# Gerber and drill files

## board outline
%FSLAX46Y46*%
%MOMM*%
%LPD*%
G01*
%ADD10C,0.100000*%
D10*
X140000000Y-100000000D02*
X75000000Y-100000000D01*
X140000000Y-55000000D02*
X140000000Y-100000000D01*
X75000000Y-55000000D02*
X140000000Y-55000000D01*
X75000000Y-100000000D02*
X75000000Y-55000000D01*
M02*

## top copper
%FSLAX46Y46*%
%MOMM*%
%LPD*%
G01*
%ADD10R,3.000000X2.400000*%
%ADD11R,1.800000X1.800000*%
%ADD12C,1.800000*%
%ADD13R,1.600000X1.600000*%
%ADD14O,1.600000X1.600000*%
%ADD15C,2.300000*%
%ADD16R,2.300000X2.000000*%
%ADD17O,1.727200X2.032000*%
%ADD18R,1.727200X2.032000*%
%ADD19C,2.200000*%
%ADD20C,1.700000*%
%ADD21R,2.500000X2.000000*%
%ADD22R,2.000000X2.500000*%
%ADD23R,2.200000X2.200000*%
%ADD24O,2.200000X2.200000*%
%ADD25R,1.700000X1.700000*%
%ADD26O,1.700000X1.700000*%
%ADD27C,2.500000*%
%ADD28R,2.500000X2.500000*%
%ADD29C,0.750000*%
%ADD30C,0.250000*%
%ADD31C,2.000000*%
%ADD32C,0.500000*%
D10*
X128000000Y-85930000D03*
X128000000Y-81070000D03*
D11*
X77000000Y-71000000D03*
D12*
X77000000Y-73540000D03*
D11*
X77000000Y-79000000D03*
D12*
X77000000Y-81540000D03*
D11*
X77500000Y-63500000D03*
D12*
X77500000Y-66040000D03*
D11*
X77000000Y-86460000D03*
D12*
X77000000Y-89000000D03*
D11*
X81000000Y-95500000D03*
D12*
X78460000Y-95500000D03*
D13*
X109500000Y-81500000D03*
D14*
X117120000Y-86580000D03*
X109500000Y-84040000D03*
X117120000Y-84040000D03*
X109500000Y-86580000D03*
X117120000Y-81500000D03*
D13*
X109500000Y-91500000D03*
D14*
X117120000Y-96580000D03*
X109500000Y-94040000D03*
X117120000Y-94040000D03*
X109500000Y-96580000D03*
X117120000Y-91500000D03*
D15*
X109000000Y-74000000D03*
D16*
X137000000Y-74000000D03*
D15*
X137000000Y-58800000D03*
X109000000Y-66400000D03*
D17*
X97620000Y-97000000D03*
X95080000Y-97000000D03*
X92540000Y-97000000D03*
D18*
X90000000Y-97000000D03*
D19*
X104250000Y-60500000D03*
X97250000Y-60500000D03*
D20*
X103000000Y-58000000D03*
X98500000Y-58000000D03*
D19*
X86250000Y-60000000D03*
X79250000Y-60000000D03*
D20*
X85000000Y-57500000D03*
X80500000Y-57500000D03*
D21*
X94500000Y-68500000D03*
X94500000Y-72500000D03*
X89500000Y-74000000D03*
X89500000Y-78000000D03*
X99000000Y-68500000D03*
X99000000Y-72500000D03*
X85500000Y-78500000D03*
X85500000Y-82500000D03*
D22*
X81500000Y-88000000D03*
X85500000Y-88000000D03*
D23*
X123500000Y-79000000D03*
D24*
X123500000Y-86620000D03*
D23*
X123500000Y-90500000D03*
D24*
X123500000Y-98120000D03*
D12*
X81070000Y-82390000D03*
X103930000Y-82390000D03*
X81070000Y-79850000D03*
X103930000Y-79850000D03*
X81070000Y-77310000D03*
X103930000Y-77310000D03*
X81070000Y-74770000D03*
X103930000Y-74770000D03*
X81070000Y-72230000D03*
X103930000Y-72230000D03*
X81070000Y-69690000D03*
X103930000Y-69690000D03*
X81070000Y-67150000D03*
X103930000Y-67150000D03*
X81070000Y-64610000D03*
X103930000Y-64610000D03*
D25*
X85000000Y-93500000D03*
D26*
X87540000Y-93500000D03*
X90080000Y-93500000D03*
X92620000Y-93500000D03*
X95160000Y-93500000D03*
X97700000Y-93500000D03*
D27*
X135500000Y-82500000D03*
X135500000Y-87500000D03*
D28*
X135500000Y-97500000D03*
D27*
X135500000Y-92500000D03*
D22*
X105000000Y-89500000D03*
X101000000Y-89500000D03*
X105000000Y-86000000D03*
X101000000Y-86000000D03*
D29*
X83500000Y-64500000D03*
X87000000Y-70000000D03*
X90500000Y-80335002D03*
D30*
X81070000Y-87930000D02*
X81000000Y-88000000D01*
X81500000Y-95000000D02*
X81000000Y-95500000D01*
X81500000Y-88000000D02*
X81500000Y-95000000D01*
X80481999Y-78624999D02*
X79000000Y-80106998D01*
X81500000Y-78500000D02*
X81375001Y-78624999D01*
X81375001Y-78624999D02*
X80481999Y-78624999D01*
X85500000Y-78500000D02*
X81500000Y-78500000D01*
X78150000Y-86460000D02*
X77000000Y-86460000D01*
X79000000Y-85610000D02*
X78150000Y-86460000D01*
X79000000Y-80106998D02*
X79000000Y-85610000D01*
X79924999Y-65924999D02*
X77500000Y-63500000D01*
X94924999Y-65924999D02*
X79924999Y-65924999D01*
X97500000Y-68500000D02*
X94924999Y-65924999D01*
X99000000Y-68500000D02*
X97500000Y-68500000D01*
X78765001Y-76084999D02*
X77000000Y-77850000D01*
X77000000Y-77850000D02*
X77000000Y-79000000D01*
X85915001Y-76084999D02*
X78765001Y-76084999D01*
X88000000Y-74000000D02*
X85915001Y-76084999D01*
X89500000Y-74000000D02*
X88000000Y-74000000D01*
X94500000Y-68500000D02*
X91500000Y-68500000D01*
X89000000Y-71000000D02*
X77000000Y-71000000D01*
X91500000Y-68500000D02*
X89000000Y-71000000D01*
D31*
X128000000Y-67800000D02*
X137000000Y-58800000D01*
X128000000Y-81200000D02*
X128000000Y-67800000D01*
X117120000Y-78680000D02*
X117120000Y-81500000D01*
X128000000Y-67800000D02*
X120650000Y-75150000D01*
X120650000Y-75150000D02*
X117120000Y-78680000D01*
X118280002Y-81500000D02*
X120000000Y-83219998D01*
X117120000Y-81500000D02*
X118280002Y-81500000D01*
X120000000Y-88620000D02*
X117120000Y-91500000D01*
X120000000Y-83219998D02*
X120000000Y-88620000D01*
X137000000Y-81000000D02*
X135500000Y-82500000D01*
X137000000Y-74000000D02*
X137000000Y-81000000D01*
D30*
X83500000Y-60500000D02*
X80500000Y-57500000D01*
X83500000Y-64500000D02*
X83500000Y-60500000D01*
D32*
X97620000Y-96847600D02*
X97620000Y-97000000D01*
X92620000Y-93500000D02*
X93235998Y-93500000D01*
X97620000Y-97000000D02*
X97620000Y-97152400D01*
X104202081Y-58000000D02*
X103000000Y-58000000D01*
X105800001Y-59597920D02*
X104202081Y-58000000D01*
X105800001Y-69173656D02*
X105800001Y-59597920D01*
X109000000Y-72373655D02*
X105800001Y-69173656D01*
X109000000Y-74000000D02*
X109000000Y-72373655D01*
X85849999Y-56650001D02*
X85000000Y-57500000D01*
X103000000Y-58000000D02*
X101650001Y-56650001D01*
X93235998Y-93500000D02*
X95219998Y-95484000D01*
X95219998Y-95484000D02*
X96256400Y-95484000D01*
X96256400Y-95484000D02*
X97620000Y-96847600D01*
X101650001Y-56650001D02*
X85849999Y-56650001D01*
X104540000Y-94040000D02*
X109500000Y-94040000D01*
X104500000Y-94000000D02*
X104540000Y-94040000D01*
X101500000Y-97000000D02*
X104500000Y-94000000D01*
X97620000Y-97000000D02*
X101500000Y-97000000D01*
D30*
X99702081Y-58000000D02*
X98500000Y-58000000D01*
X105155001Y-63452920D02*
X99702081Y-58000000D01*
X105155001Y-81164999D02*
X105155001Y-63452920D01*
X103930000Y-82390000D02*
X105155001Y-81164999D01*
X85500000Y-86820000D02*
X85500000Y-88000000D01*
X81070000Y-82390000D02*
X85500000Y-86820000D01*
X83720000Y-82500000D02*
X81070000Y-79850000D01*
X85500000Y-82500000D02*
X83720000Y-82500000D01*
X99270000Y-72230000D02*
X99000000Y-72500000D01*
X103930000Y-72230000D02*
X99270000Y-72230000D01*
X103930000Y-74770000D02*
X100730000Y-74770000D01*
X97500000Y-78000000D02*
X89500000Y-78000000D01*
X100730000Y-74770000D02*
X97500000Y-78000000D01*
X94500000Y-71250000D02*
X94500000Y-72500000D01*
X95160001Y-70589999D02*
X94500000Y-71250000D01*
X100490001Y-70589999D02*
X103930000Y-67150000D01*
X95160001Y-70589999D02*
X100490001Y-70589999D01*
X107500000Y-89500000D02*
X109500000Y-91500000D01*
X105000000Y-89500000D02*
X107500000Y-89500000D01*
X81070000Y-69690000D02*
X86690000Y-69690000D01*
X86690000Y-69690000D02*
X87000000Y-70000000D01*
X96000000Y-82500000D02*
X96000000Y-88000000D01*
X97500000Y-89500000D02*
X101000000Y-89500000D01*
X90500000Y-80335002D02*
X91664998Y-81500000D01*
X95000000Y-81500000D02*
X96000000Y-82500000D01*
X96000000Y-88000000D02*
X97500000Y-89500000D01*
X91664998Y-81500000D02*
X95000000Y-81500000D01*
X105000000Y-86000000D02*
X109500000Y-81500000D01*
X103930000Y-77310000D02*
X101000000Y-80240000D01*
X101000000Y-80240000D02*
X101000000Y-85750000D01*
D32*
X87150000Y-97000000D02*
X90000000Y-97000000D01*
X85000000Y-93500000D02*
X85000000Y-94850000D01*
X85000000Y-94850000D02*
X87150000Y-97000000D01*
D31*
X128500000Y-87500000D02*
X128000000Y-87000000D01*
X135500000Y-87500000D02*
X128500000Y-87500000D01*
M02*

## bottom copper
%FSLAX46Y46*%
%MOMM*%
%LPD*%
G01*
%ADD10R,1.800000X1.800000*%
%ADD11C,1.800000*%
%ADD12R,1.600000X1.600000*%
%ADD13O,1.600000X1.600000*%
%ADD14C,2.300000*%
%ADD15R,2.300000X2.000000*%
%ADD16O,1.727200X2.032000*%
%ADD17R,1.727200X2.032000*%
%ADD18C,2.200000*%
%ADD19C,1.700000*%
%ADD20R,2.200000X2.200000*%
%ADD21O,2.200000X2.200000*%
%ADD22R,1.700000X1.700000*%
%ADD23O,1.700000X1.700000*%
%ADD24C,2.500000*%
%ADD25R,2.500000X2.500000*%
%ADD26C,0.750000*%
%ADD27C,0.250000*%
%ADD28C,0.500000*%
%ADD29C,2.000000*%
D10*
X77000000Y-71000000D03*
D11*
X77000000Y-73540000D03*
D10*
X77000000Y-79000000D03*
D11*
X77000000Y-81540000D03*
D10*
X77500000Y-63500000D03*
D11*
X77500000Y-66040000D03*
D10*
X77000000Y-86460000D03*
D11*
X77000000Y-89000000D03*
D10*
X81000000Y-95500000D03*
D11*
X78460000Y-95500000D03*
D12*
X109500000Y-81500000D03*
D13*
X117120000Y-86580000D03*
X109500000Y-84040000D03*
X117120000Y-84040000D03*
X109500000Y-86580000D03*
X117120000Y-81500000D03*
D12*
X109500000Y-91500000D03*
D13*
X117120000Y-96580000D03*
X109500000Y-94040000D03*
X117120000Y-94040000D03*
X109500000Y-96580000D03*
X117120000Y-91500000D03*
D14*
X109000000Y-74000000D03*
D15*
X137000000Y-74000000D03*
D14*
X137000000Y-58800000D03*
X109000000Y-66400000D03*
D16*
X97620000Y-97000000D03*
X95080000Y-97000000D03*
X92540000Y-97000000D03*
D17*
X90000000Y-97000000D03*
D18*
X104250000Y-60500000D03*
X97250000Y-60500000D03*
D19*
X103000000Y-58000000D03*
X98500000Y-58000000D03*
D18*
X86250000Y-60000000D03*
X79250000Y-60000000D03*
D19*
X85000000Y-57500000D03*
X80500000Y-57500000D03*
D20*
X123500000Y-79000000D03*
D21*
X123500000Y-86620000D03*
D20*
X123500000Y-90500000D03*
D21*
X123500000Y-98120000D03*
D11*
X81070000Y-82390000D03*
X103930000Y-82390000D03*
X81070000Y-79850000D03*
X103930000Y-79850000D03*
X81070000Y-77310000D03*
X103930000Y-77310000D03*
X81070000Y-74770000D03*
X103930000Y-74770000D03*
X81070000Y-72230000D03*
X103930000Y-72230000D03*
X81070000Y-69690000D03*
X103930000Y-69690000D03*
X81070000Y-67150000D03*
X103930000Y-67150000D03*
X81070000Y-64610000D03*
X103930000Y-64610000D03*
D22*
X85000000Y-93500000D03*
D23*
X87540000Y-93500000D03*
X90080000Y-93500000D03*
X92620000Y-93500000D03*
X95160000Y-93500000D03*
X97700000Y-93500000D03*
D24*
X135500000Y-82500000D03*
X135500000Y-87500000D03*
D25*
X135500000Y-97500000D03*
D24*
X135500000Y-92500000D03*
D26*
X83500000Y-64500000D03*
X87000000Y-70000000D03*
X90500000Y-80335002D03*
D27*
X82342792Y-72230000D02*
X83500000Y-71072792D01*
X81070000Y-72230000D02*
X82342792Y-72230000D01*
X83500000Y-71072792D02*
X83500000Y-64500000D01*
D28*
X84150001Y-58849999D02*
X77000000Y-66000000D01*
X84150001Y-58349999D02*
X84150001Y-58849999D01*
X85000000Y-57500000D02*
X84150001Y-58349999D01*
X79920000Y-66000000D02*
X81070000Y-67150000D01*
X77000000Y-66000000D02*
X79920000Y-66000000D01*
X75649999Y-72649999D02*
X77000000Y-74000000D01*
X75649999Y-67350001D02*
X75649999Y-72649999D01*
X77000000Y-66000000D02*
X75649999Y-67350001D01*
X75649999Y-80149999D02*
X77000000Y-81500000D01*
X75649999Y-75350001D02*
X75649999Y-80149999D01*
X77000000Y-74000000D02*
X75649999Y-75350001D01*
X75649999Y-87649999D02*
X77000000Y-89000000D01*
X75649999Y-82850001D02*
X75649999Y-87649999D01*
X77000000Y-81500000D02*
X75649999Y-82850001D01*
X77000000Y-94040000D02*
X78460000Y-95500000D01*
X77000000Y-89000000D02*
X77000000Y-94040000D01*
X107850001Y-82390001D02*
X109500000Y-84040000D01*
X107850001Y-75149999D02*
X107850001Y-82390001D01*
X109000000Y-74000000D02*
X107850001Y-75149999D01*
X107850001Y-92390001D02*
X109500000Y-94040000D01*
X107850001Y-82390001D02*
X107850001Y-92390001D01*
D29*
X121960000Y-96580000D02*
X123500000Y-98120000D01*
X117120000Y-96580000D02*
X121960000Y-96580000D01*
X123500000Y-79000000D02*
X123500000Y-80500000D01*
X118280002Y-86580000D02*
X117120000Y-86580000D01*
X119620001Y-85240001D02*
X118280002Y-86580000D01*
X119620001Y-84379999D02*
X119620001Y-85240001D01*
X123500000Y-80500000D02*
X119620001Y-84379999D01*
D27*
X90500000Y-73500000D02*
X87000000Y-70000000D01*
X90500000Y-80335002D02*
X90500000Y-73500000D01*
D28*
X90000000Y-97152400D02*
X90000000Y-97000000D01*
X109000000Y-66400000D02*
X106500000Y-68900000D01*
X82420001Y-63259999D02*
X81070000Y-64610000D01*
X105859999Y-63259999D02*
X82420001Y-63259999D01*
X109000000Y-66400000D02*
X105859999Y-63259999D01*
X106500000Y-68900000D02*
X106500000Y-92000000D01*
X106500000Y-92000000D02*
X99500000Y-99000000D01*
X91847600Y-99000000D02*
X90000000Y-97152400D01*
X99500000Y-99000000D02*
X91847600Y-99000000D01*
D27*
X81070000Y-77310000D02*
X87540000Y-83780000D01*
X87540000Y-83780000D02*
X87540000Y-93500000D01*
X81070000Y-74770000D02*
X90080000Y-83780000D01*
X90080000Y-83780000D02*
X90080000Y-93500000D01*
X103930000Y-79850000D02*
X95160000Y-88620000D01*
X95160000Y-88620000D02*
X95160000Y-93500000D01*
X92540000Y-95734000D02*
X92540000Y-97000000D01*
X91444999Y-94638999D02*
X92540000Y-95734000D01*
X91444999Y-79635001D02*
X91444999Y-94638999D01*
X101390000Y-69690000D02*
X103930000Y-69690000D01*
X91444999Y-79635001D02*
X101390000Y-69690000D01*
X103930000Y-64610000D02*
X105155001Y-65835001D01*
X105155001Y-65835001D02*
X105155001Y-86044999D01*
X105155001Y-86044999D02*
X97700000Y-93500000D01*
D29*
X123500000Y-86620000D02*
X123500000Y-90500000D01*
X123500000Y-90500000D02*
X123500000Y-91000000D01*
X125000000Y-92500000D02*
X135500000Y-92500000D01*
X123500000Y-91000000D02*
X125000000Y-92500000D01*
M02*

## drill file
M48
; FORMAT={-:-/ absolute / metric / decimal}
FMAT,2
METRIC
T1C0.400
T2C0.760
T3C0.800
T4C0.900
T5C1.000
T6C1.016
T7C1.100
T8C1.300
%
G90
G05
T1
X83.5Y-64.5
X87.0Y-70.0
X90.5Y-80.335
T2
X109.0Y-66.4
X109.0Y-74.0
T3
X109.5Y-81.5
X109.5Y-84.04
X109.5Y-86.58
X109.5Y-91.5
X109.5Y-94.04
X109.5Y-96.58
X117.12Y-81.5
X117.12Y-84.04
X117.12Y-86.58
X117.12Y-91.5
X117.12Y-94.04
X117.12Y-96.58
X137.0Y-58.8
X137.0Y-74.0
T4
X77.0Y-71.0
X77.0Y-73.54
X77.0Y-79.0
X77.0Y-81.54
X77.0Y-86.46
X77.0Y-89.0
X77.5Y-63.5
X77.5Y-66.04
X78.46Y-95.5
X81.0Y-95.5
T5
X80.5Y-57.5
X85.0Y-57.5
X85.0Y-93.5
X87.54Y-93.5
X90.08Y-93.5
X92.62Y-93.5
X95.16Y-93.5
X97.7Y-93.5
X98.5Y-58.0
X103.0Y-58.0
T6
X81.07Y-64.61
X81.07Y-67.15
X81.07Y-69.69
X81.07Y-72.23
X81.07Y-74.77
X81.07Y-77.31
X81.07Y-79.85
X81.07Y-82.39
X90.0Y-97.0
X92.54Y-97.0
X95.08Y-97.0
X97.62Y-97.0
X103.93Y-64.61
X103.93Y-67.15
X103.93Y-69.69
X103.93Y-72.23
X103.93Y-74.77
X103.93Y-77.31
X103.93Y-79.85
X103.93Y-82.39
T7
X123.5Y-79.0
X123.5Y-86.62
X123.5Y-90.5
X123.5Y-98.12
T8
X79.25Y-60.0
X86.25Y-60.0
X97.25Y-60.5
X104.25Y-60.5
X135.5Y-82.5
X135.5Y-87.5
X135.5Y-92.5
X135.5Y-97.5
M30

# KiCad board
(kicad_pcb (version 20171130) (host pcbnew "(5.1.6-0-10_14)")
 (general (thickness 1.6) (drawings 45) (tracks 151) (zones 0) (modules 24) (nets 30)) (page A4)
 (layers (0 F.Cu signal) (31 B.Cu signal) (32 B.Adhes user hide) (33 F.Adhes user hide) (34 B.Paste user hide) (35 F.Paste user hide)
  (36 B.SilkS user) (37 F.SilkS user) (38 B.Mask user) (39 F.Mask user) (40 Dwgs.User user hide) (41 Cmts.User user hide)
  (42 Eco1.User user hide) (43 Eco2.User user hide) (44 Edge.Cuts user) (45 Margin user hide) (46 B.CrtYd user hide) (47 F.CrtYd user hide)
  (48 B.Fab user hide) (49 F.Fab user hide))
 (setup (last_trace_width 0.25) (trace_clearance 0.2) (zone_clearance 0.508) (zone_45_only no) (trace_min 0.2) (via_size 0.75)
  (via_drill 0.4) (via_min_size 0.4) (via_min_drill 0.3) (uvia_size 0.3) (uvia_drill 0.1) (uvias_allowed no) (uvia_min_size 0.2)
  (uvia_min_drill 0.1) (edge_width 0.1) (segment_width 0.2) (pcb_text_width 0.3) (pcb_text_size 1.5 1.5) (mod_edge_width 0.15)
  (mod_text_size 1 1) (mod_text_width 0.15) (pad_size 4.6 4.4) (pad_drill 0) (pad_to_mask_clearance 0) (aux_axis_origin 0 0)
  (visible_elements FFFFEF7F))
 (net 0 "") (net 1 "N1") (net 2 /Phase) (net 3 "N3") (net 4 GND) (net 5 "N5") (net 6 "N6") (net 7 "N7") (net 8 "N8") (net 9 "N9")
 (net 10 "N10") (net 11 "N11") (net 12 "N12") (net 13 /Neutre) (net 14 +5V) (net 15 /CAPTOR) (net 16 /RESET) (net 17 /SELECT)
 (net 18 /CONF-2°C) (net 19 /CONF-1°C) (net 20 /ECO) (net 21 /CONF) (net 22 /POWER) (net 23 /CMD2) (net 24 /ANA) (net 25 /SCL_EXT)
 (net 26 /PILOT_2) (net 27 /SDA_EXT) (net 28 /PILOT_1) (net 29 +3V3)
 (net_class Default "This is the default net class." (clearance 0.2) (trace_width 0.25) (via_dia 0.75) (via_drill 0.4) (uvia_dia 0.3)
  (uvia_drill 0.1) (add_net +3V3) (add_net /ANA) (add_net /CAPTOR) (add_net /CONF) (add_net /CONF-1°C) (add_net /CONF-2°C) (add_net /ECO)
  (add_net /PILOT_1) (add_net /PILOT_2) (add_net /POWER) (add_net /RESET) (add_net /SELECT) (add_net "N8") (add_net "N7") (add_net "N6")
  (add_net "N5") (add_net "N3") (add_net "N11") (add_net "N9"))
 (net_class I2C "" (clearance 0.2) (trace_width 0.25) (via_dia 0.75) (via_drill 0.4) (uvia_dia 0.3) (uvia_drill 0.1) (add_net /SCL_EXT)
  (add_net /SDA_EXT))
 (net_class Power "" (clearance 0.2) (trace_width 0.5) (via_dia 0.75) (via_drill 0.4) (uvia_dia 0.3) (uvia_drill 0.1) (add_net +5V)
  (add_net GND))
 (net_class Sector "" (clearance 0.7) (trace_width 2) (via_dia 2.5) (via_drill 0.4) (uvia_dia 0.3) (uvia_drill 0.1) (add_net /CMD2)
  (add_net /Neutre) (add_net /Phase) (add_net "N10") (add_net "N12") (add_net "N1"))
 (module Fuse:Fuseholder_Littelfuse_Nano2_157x (layer F.Cu) (at 128 83.5 270)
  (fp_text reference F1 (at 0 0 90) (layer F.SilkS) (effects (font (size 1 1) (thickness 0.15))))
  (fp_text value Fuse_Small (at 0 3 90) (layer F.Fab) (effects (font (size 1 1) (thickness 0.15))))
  (pad 2 smd rect (at 2.43 0 270) (size 2.4 3) (layers F.Cu F.Paste F.Mask) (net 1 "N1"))
  (pad 1 smd rect (at -2.43 0 270) (size 2.4 3) (layers F.Cu F.Paste F.Mask) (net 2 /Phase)))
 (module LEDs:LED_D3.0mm (layer F.Cu) (at 77 71 270)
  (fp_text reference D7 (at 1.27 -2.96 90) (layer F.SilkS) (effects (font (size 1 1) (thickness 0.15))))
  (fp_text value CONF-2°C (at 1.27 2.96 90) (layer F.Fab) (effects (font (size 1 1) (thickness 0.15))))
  (pad 1 thru_hole rect (at 0 0 270) (size 1.8 1.8) (drill 0.9) (layers *.Cu *.Mask) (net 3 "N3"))
  (pad 2 thru_hole circle (at 2.54 0 270) (size 1.8 1.8) (drill 0.9) (layers *.Cu *.Mask) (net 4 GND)))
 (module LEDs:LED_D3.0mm (layer F.Cu) (at 77 79 270)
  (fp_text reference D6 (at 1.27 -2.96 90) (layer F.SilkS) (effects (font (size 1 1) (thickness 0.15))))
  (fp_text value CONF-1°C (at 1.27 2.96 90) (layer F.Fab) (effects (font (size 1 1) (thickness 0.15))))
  (pad 1 thru_hole rect (at 0 0 270) (size 1.8 1.8) (drill 0.9) (layers *.Cu *.Mask) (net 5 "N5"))
  (pad 2 thru_hole circle (at 2.54 0 270) (size 1.8 1.8) (drill 0.9) (layers *.Cu *.Mask) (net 4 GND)))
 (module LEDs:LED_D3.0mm (layer F.Cu) (at 77.5 63.5 270)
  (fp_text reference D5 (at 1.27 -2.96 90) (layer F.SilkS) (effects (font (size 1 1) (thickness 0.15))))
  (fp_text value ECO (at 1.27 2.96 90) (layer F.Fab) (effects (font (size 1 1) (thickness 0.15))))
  (pad 1 thru_hole rect (at 0 0 270) (size 1.8 1.8) (drill 0.9) (layers *.Cu *.Mask) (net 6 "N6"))
  (pad 2 thru_hole circle (at 2.54 0 270) (size 1.8 1.8) (drill 0.9) (layers *.Cu *.Mask) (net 4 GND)))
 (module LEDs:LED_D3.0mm (layer F.Cu) (at 77 86.46 270)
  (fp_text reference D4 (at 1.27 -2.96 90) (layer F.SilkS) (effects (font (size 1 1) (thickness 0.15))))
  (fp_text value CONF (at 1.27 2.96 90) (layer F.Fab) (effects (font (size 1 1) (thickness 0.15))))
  (pad 1 thru_hole rect (at 0 0 270) (size 1.8 1.8) (drill 0.9) (layers *.Cu *.Mask) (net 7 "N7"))
  (pad 2 thru_hole circle (at 2.54 0 270) (size 1.8 1.8) (drill 0.9) (layers *.Cu *.Mask) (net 4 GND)))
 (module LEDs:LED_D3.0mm (layer F.Cu) (at 81 95.5 180)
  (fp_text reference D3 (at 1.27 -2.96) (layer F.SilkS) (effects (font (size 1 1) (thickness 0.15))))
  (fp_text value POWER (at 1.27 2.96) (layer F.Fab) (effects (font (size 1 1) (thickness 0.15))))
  (pad 1 thru_hole rect (at 0 0 180) (size 1.8 1.8) (drill 0.9) (layers *.Cu *.Mask) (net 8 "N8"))
  (pad 2 thru_hole circle (at 2.54 0 180) (size 1.8 1.8) (drill 0.9) (layers *.Cu *.Mask) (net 4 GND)))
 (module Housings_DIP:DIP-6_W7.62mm (layer F.Cu) (at 109.5 81.5)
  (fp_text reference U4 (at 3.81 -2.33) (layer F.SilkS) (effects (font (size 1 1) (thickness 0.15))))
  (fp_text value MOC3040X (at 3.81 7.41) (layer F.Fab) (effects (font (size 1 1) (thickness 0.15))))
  (pad 1 thru_hole rect (at 0 0) (size 1.6 1.6) (drill 0.8) (layers *.Cu *.Mask) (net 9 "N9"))
  (pad 4 thru_hole oval (at 7.62 5.08) (size 1.6 1.6) (drill 0.8) (layers *.Cu *.Mask) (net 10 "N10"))
  (pad 2 thru_hole oval (at 0 2.54) (size 1.6 1.6) (drill 0.8) (layers *.Cu *.Mask) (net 4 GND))
  (pad 5 thru_hole oval (at 7.62 2.54) (size 1.6 1.6) (drill 0.8) (layers *.Cu *.Mask))
  (pad 3 thru_hole oval (at 0 5.08) (size 1.6 1.6) (drill 0.8) (layers *.Cu *.Mask))
  (pad 6 thru_hole oval (at 7.62 0) (size 1.6 1.6) (drill 0.8) (layers *.Cu *.Mask) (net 2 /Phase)))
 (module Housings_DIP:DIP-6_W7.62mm (layer F.Cu) (at 109.5 91.5)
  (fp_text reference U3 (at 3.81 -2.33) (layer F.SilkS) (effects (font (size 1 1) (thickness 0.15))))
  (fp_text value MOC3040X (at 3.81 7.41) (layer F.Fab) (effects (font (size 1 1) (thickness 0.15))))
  (pad 1 thru_hole rect (at 0 0) (size 1.6 1.6) (drill 0.8) (layers *.Cu *.Mask) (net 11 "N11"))
  (pad 4 thru_hole oval (at 7.62 5.08) (size 1.6 1.6) (drill 0.8) (layers *.Cu *.Mask) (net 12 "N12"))
  (pad 2 thru_hole oval (at 0 2.54) (size 1.6 1.6) (drill 0.8) (layers *.Cu *.Mask) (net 4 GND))
  (pad 5 thru_hole oval (at 7.62 2.54) (size 1.6 1.6) (drill 0.8) (layers *.Cu *.Mask))
  (pad 3 thru_hole oval (at 0 5.08) (size 1.6 1.6) (drill 0.8) (layers *.Cu *.Mask))
  (pad 6 thru_hole oval (at 7.62 0) (size 1.6 1.6) (drill 0.8) (layers *.Cu *.Mask) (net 2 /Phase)))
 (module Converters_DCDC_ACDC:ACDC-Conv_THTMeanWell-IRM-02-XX (layer F.Cu) (at 137 74 180)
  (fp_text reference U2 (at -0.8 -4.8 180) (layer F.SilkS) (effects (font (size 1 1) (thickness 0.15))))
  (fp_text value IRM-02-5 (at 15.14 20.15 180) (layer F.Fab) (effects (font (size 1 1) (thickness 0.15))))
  (pad 3 thru_hole circle (at 28 0 180) (size 2.3 2.3) (drill 0.76) (layers *.Cu *.Mask) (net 4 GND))
  (pad 1 thru_hole rect (at 0 0 180) (size 2.3 2) (drill 0.8) (layers *.Cu *.Mask) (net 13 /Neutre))
  (pad 2 thru_hole circle (at 0 15.2 180) (size 2.3 2.3) (drill 0.8) (layers *.Cu *.Mask) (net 2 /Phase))
  (pad 4 thru_hole circle (at 28 7.6 180) (size 2.3 2.3) (drill 0.76) (layers *.Cu *.Mask) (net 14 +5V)))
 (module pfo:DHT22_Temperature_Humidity (layer F.Cu) (at 93.81 97)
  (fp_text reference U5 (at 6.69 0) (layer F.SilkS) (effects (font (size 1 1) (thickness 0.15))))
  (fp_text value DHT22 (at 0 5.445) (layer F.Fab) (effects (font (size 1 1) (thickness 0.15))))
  (pad 4 thru_hole oval (at 3.81 0 90) (size 2.032 1.7272) (drill 1.016) (layers *.Cu *.Mask F.SilkS) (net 4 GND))
  (pad 3 thru_hole oval (at 1.27 0 90) (size 2.032 1.7272) (drill 1.016) (layers *.Cu *.Mask F.SilkS))
  (pad 2 thru_hole oval (at -1.27 0 90) (size 2.032 1.7272) (drill 1.016) (layers *.Cu *.Mask F.SilkS) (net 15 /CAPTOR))
  (pad 1 thru_hole rect (at -3.81 0 90) (size 2.032 1.7272) (drill 1.016) (layers *.Cu *.Mask F.SilkS) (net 14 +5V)))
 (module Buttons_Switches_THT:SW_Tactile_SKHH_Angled (layer F.Cu) (at 98.5 58)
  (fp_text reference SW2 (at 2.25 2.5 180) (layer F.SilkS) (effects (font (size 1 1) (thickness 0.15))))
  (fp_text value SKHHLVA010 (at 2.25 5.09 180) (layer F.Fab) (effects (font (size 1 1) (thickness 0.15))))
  (pad "" thru_hole circle (at 5.75 2.5 180) (size 2.2 2.2) (drill 1.3) (layers *.Cu *.Mask))
  (pad "" thru_hole circle (at -1.25 2.5 180) (size 2.2 2.2) (drill 1.3) (layers *.Cu *.Mask))
  (pad 2 thru_hole circle (at 4.5 0 180) (size 1.7 1.7) (drill 1) (layers *.Cu *.Mask) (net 4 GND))
  (pad 1 thru_hole circle (at 0 0 180) (size 1.7 1.7) (drill 1) (layers *.Cu *.Mask) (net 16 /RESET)))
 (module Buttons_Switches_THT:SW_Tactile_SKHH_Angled (layer F.Cu) (at 80.5 57.5)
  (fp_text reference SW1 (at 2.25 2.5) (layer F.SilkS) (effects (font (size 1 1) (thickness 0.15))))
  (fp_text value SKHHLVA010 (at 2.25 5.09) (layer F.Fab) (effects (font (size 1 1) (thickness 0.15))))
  (pad "" thru_hole circle (at 5.75 2.5 180) (size 2.2 2.2) (drill 1.3) (layers *.Cu *.Mask))
  (pad "" thru_hole circle (at -1.25 2.5 180) (size 2.2 2.2) (drill 1.3) (layers *.Cu *.Mask))
  (pad 2 thru_hole circle (at 4.5 0 180) (size 1.7 1.7) (drill 1) (layers *.Cu *.Mask) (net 4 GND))
  (pad 1 thru_hole circle (at 0 0 180) (size 1.7 1.7) (drill 1) (layers *.Cu *.Mask) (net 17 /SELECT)))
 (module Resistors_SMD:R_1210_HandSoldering (layer F.Cu) (at 94.5 70.5 270)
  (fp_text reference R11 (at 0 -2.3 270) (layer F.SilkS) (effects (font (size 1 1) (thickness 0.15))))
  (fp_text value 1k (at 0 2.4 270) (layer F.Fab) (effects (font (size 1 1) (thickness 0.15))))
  (pad 1 smd rect (at -2 0 270) (size 2 2.5) (layers F.Cu F.Paste F.Mask) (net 3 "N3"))
  (pad 2 smd rect (at 2 0 270) (size 2 2.5) (layers F.Cu F.Paste F.Mask) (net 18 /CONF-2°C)))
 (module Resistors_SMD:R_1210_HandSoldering (layer F.Cu) (at 89.5 76 270)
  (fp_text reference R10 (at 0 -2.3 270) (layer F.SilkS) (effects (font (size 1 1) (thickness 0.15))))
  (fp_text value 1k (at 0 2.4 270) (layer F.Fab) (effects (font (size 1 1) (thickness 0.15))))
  (pad 1 smd rect (at -2 0 270) (size 2 2.5) (layers F.Cu F.Paste F.Mask) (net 5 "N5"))
  (pad 2 smd rect (at 2 0 270) (size 2 2.5) (layers F.Cu F.Paste F.Mask) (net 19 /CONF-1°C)))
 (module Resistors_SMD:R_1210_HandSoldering (layer F.Cu) (at 99 70.5 270)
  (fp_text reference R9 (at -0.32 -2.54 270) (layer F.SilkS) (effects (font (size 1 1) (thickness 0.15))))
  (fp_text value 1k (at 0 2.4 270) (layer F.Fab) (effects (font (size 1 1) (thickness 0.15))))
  (pad 1 smd rect (at -2 0 270) (size 2 2.5) (layers F.Cu F.Paste F.Mask) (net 6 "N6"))
  (pad 2 smd rect (at 2 0 270) (size 2 2.5) (layers F.Cu F.Paste F.Mask) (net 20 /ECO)))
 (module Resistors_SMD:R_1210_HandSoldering (layer F.Cu) (at 85.5 80.5 270)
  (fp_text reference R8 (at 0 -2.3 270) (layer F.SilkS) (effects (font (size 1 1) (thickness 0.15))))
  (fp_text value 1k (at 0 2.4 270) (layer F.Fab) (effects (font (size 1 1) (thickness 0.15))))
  (pad 1 smd rect (at -2 0 270) (size 2 2.5) (layers F.Cu F.Paste F.Mask) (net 7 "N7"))
  (pad 2 smd rect (at 2 0 270) (size 2 2.5) (layers F.Cu F.Paste F.Mask) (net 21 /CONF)))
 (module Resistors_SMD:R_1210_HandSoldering (layer F.Cu) (at 83.5 88)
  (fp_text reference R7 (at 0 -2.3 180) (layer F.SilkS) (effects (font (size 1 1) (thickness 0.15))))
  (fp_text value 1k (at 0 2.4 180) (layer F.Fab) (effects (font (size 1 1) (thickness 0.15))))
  (pad 1 smd rect (at -2 0) (size 2 2.5) (layers F.Cu F.Paste F.Mask) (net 8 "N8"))
  (pad 2 smd rect (at 2 0) (size 2 2.5) (layers F.Cu F.Paste F.Mask) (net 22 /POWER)))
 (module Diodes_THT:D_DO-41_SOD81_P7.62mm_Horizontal (layer F.Cu) (at 123.5 79 270)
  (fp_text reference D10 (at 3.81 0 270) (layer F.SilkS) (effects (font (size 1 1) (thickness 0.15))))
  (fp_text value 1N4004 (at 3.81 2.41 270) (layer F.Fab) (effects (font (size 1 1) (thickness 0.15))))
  (pad 1 thru_hole rect (at 0 0 270) (size 2.2 2.2) (drill 1.1) (layers *.Cu *.Mask) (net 10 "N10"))
  (pad 2 thru_hole oval (at 7.62 0 270) (size 2.2 2.2) (drill 1.1) (layers *.Cu *.Mask) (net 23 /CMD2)))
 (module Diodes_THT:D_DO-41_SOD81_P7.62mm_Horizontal (layer F.Cu) (at 123.5 90.5 270)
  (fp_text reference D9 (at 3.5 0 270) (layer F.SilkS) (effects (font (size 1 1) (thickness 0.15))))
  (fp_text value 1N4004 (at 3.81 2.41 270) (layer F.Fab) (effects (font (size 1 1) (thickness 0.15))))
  (pad 1 thru_hole rect (at 0 0 270) (size 2.2 2.2) (drill 1.1) (layers *.Cu *.Mask) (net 23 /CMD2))
  (pad 2 thru_hole oval (at 7.62 0 270) (size 2.2 2.2) (drill 1.1) (layers *.Cu *.Mask) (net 12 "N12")))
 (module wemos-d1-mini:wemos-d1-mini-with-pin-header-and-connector (layer F.Cu) (at 92.5 73.5 270)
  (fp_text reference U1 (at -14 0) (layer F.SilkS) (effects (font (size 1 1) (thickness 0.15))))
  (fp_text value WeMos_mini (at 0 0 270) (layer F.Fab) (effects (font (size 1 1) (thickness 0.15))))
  (pad 8 thru_hole circle (at 8.89 11.43 270) (size 1.8 1.8) (drill 1.016) (layers *.Cu *.Mask) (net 22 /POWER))
  (pad 9 thru_hole circle (at 8.89 -11.43 270) (size 1.8 1.8) (drill 1.016) (layers *.Cu *.Mask) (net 16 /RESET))
  (pad 7 thru_hole circle (at 6.35 11.43 270) (size 1.8 1.8) (drill 1.016) (layers *.Cu *.Mask) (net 21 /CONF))
  (pad 10 thru_hole circle (at 6.35 -11.43 270) (size 1.8 1.8) (drill 1.016) (layers *.Cu *.Mask) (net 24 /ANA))
  (pad 6 thru_hole circle (at 3.81 11.43 270) (size 1.8 1.8) (drill 1.016) (layers *.Cu *.Mask) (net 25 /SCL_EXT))
  (pad 11 thru_hole circle (at 3.81 -11.43 270) (size 1.8 1.8) (drill 1.016) (layers *.Cu *.Mask) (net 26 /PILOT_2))
  (pad 5 thru_hole circle (at 1.27 11.43 270) (size 1.8 1.8) (drill 1.016) (layers *.Cu *.Mask) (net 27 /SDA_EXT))
  (pad 12 thru_hole circle (at 1.27 -11.43 270) (size 1.8 1.8) (drill 1.016) (layers *.Cu *.Mask) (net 19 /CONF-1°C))
  (pad 4 thru_hole circle (at -1.27 11.43 270) (size 1.8 1.8) (drill 1.016) (layers *.Cu *.Mask) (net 17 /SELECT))
  (pad 13 thru_hole circle (at -1.27 -11.43 270) (size 1.8 1.8) (drill 1.016) (layers *.Cu *.Mask) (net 20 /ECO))
  (pad 3 thru_hole circle (at -3.81 11.43 270) (size 1.8 1.8) (drill 1.016) (layers *.Cu *.Mask) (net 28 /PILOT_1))
  (pad 14 thru_hole circle (at -3.81 -11.43 270) (size 1.8 1.8) (drill 1.016) (layers *.Cu *.Mask) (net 15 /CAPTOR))
  (pad 2 thru_hole circle (at -6.35 11.43 270) (size 1.8 1.8) (drill 1.016) (layers *.Cu *.Mask) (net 4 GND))
  (pad 15 thru_hole circle (at -6.35 -11.43 270) (size 1.8 1.8) (drill 1.016) (layers *.Cu *.Mask) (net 18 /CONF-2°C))
  (pad 1 thru_hole circle (at -8.89 11.43 270) (size 1.8 1.8) (drill 1.016) (layers *.Cu *.Mask) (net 14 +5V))
  (pad 16 thru_hole circle (at -8.89 -11.43 270) (size 1.8 1.8) (drill 1.016) (layers *.Cu *.Mask) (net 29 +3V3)))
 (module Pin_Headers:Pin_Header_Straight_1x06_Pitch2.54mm (layer F.Cu) (at 85 93.5 90)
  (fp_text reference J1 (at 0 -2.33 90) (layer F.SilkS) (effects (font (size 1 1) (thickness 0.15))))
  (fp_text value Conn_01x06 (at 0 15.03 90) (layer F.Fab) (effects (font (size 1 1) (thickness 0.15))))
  (pad 1 thru_hole rect (at 0 0 90) (size 1.7 1.7) (drill 1) (layers *.Cu *.Mask) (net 14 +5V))
  (pad 2 thru_hole oval (at 0 2.54 90) (size 1.7 1.7) (drill 1) (layers *.Cu *.Mask) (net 25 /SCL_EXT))
  (pad 3 thru_hole oval (at 0 5.08 90) (size 1.7 1.7) (drill 1) (layers *.Cu *.Mask) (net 27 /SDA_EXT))
  (pad 4 thru_hole oval (at 0 7.62 90) (size 1.7 1.7) (drill 1) (layers *.Cu *.Mask) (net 4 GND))
  (pad 5 thru_hole oval (at 0 10.16 90) (size 1.7 1.7) (drill 1) (layers *.Cu *.Mask) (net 24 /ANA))
  (pad 6 thru_hole oval (at 0 12.7 90) (size 1.7 1.7) (drill 1) (layers *.Cu *.Mask) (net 29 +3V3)))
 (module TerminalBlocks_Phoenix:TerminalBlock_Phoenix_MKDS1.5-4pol (layer F.Cu) (at 135.5 97.5 90)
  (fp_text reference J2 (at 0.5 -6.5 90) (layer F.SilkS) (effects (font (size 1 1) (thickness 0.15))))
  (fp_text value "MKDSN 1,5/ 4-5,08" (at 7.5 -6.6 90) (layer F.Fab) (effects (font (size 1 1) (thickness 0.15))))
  (pad 4 thru_hole circle (at 15 0 90) (size 2.5 2.5) (drill 1.3) (layers *.Cu *.Mask) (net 13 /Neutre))
  (pad 3 thru_hole circle (at 10 0 90) (size 2.5 2.5) (drill 1.3) (layers *.Cu *.Mask) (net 1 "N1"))
  (pad 1 thru_hole rect (at 0 0 90) (size 2.5 2.5) (drill 1.3) (layers *.Cu *.Mask))
  (pad 2 thru_hole circle (at 5 0 90) (size 2.5 2.5) (drill 1.3) (layers *.Cu *.Mask) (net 23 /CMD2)))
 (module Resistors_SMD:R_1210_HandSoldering (layer F.Cu) (at 103 89.5 180)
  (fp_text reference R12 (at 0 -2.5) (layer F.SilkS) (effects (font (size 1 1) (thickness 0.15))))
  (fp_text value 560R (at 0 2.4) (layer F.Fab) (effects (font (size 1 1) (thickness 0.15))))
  (pad 1 smd rect (at -2 0 180) (size 2 2.5) (layers F.Cu F.Paste F.Mask) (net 11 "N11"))
  (pad 2 smd rect (at 2 0 180) (size 2 2.5) (layers F.Cu F.Paste F.Mask) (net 28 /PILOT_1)))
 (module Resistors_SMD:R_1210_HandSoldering (layer F.Cu) (at 103 86 180)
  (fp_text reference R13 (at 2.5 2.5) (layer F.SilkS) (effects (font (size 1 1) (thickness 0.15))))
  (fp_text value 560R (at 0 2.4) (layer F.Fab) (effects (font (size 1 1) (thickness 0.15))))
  (pad 1 smd rect (at -2 0 180) (size 2 2.5) (layers F.Cu F.Paste F.Mask) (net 9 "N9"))
  (pad 2 smd rect (at 2 0 180) (size 2 2.5) (layers F.Cu F.Paste F.Mask) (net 26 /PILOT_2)))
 (gr_line (start 140 100) (end 75 100) (layer Edge.Cuts) (width 0.1))
 (gr_line (start 140 55) (end 140 100) (layer Edge.Cuts) (width 0.1))
 (gr_line (start 75 55) (end 140 55) (layer Edge.Cuts) (width 0.1))
 (gr_line (start 75 100) (end 75 55) (layer Edge.Cuts) (width 0.1))
 (segment (start 81.07 87.93) (end 81 88) (width 0.25) (layer F.Cu) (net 8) (status 30))
 (segment (start 81.5 95) (end 81 95.5) (width 0.25) (layer F.Cu) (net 8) (status 30))
 (segment (start 81.5 88) (end 81.5 95) (width 0.25) (layer F.Cu) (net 8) (status 30))
 (segment (start 80.481999 78.624999) (end 79 80.106998) (width 0.25) (layer F.Cu) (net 7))
 (segment (start 81.5 78.5) (end 81.375001 78.624999) (width 0.25) (layer F.Cu) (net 7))
 (segment (start 81.375001 78.624999) (end 80.481999 78.624999) (width 0.25) (layer F.Cu) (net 7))
 (segment (start 85.5 78.5) (end 81.5 78.5) (width 0.25) (layer F.Cu) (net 7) (status 10))
 (segment (start 78.15 86.46) (end 77 86.46) (width 0.25) (layer F.Cu) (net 7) (status 20))
 (segment (start 79 85.61) (end 78.15 86.46) (width 0.25) (layer F.Cu) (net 7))
 (segment (start 79 80.106998) (end 79 85.61) (width 0.25) (layer F.Cu) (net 7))
 (segment (start 79.924999 65.924999) (end 77.5 63.5) (width 0.25) (layer F.Cu) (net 6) (status 20))
 (segment (start 94.924999 65.924999) (end 79.924999 65.924999) (width 0.25) (layer F.Cu) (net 6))
 (segment (start 97.5 68.5) (end 94.924999 65.924999) (width 0.25) (layer F.Cu) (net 6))
 (segment (start 99 68.5) (end 97.5 68.5) (width 0.25) (layer F.Cu) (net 6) (status 10))
 (segment (start 78.765001 76.084999) (end 77 77.85) (width 0.25) (layer F.Cu) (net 5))
 (segment (start 77 77.85) (end 77 79) (width 0.25) (layer F.Cu) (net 5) (status 20))
 (segment (start 85.915001 76.084999) (end 78.765001 76.084999) (width 0.25) (layer F.Cu) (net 5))
 (segment (start 88 74) (end 85.915001 76.084999) (width 0.25) (layer F.Cu) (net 5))
 (segment (start 89.5 74) (end 88 74) (width 0.25) (layer F.Cu) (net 5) (status 10))
 (segment (start 94.5 68.5) (end 91.5 68.5) (width 0.25) (layer F.Cu) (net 3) (status 10))
 (segment (start 89 71) (end 77 71) (width 0.25) (layer F.Cu) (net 3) (status 20))
 (segment (start 91.5 68.5) (end 89 71) (width 0.25) (layer F.Cu) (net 3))
 (segment (start 128 67.8) (end 137 58.8) (width 2) (layer F.Cu) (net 2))
 (segment (start 128 81.2) (end 128 67.8) (width 2) (layer F.Cu) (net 2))
 (segment (start 117.12 78.68) (end 117.12 81.5) (width 2) (layer F.Cu) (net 2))
 (segment (start 128 67.8) (end 120.65 75.15) (width 2) (layer F.Cu) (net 2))
 (segment (start 120.65 75.15) (end 117.12 78.68) (width 2) (layer F.Cu) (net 2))
 (segment (start 118.280002 81.5) (end 120 83.219998) (width 2) (layer F.Cu) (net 2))
 (segment (start 117.12 81.5) (end 118.280002 81.5) (width 2) (layer F.Cu) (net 2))
 (segment (start 120 88.62) (end 117.12 91.5) (width 2) (layer F.Cu) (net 2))
 (segment (start 120 83.219998) (end 120 88.62) (width 2) (layer F.Cu) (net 2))
 (segment (start 137 81) (end 135.5 82.5) (width 2) (layer F.Cu) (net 13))
 (segment (start 137 74) (end 137 81) (width 2) (layer F.Cu) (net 13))
 (segment (start 82.342792 72.23) (end 83.5 71.072792) (width 0.25) (layer B.Cu) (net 17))
 (segment (start 81.07 72.23) (end 82.342792 72.23) (width 0.25) (layer B.Cu) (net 17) (status 10))
 (segment (start 83.5 71.072792) (end 83.5 64.5) (width 0.25) (layer B.Cu) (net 17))
 (via (at 83.5 64.5) (size 0.75) (drill 0.4) (layers F.Cu B.Cu) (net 17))
 (segment (start 83.5 60.5) (end 80.5 57.5) (width 0.25) (layer F.Cu) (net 17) (status 20))
 (segment (start 83.5 64.5) (end 83.5 60.5) (width 0.25) (layer F.Cu) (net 17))
 (segment (start 97.62 96.8476) (end 97.62 97) (width 0.5) (layer F.Cu) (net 4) (status 30))
 (segment (start 92.62 93.5) (end 93.235998 93.5) (width 0.5) (layer F.Cu) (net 4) (status 30))
 (segment (start 97.62 97) (end 97.62 97.1524) (width 0.5) (layer F.Cu) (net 4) (status 30))
 (segment (start 104.202081 58) (end 103 58) (width 0.5) (layer F.Cu) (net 4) (status 20))
 (segment (start 105.800001 59.59792) (end 104.202081 58) (width 0.5) (layer F.Cu) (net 4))
 (segment (start 105.800001 69.173656) (end 105.800001 59.59792) (width 0.5) (layer F.Cu) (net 4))
 (segment (start 109 72.373655) (end 105.800001 69.173656) (width 0.5) (layer F.Cu) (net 4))
 (segment (start 109 74) (end 109 72.373655) (width 0.5) (layer F.Cu) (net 4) (status 10))
 (segment (start 85.849999 56.650001) (end 85 57.5) (width 0.5) (layer F.Cu) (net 4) (status 20))
 (segment (start 103 58) (end 101.650001 56.650001) (width 0.5) (layer F.Cu) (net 4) (status 10))
 (segment (start 84.150001 58.849999) (end 77 66) (width 0.5) (layer B.Cu) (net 4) (status 20))
 (segment (start 84.150001 58.349999) (end 84.150001 58.849999) (width 0.5) (layer B.Cu) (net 4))
 (segment (start 85 57.5) (end 84.150001 58.349999) (width 0.5) (layer B.Cu) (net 4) (status 10))
 (segment (start 79.92 66) (end 81.07 67.15) (width 0.5) (layer B.Cu) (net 4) (status 20))
 (segment (start 77 66) (end 79.92 66) (width 0.5) (layer B.Cu) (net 4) (status 10))
 (segment (start 75.649999 72.649999) (end 77 74) (width 0.5) (layer B.Cu) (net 4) (status 20))
 (segment (start 75.649999 67.350001) (end 75.649999 72.649999) (width 0.5) (layer B.Cu) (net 4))
 (segment (start 77 66) (end 75.649999 67.350001) (width 0.5) (layer B.Cu) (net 4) (status 10))
 (segment (start 75.649999 80.149999) (end 77 81.5) (width 0.5) (layer B.Cu) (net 4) (status 20))
 (segment (start 75.649999 75.350001) (end 75.649999 80.149999) (width 0.5) (layer B.Cu) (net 4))
 (segment (start 77 74) (end 75.649999 75.350001) (width 0.5) (layer B.Cu) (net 4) (status 10))
 (segment (start 75.649999 87.649999) (end 77 89) (width 0.5) (layer B.Cu) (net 4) (status 20))
 (segment (start 75.649999 82.850001) (end 75.649999 87.649999) (width 0.5) (layer B.Cu) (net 4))
 (segment (start 77 81.5) (end 75.649999 82.850001) (width 0.5) (layer B.Cu) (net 4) (status 10))
 (segment (start 93.235998 93.5) (end 95.219998 95.484) (width 0.5) (layer F.Cu) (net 4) (status 10))
 (segment (start 95.219998 95.484) (end 96.2564 95.484) (width 0.5) (layer F.Cu) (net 4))
 (segment (start 96.2564 95.484) (end 97.62 96.8476) (width 0.5) (layer F.Cu) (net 4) (status 20))
 (segment (start 101.650001 56.650001) (end 85.849999 56.650001) (width 0.5) (layer F.Cu) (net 4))
 (segment (start 77 94.04) (end 78.46 95.5) (width 0.5) (layer B.Cu) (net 4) (status 20))
 (segment (start 77 89) (end 77 94.04) (width 0.5) (layer B.Cu) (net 4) (status 10))
 (segment (start 104.54 94.04) (end 109.5 94.04) (width 0.5) (layer F.Cu) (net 4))
 (segment (start 104.5 94) (end 104.54 94.04) (width 0.5) (layer F.Cu) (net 4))
 (segment (start 101.5 97) (end 104.5 94) (width 0.5) (layer F.Cu) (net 4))
 (segment (start 97.62 97) (end 101.5 97) (width 0.5) (layer F.Cu) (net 4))
 (segment (start 107.850001 82.390001) (end 109.5 84.04) (width 0.5) (layer B.Cu) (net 4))
 (segment (start 107.850001 75.149999) (end 107.850001 82.390001) (width 0.5) (layer B.Cu) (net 4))
 (segment (start 109 74) (end 107.850001 75.149999) (width 0.5) (layer B.Cu) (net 4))
 (segment (start 107.850001 92.390001) (end 109.5 94.04) (width 0.5) (layer B.Cu) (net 4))
 (segment (start 107.850001 82.390001) (end 107.850001 92.390001) (width 0.5) (layer B.Cu) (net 4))
 (segment (start 99.702081 58) (end 98.5 58) (width 0.25) (layer F.Cu) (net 16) (status 20))
 (segment (start 105.155001 63.45292) (end 99.702081 58) (width 0.25) (layer F.Cu) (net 16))
 (segment (start 105.155001 81.164999) (end 105.155001 63.45292) (width 0.25) (layer F.Cu) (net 16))
 (segment (start 103.93 82.39) (end 105.155001 81.164999) (width 0.25) (layer F.Cu) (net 16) (status 10))
 (segment (start 85.5 86.82) (end 85.5 88) (width 0.25) (layer F.Cu) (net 22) (status 30))
 (segment (start 81.07 82.39) (end 85.5 86.82) (width 0.25) (layer F.Cu) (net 22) (status 30))
 (segment (start 83.72 82.5) (end 81.07 79.85) (width 0.25) (layer F.Cu) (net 21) (status 20))
 (segment (start 85.5 82.5) (end 83.72 82.5) (width 0.25) (layer F.Cu) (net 21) (status 10))
 (segment (start 99.27 72.23) (end 99 72.5) (width 0.25) (layer F.Cu) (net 20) (status 30))
 (segment (start 103.93 72.23) (end 99.27 72.23) (width 0.25) (layer F.Cu) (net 20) (status 30))
 (segment (start 103.93 74.77) (end 100.73 74.77) (width 0.25) (layer F.Cu) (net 19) (status 10))
 (segment (start 97.5 78) (end 89.5 78) (width 0.25) (layer F.Cu) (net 19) (status 20))
 (segment (start 100.73 74.77) (end 97.5 78) (width 0.25) (layer F.Cu) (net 19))
 (segment (start 94.5 71.25) (end 94.5 72.5) (width 0.25) (layer F.Cu) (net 18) (status 20))
 (segment (start 95.160001 70.589999) (end 94.5 71.25) (width 0.25) (layer F.Cu) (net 18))
 (segment (start 100.490001 70.589999) (end 103.93 67.15) (width 0.25) (layer F.Cu) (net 18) (status 20))
 (segment (start 95.160001 70.589999) (end 100.490001 70.589999) (width 0.25) (layer F.Cu) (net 18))
 (segment (start 121.96 96.58) (end 123.5 98.12) (width 2) (layer B.Cu) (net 12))
 (segment (start 117.12 96.58) (end 121.96 96.58) (width 2) (layer B.Cu) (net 12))
 (segment (start 123.5 79) (end 123.5 80.5) (width 2) (layer B.Cu) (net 10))
 (segment (start 118.280002 86.58) (end 117.12 86.58) (width 2) (layer B.Cu) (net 10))
 (segment (start 119.620001 85.240001) (end 118.280002 86.58) (width 2) (layer B.Cu) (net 10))
 (segment (start 119.620001 84.379999) (end 119.620001 85.240001) (width 2) (layer B.Cu) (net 10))
 (segment (start 123.5 80.5) (end 119.620001 84.379999) (width 2) (layer B.Cu) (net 10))
 (segment (start 107.5 89.5) (end 109.5 91.5) (width 0.25) (layer F.Cu) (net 11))
 (segment (start 105 89.5) (end 107.5 89.5) (width 0.25) (layer F.Cu) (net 11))
 (segment (start 81.07 69.69) (end 86.69 69.69) (width 0.25) (layer F.Cu) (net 28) (status 10))
 (segment (start 86.69 69.69) (end 87 70) (width 0.25) (layer F.Cu) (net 28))
 (via (at 87 70) (size 0.75) (drill 0.4) (layers F.Cu B.Cu) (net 28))
 (segment (start 90.5 73.5) (end 87 70) (width 0.25) (layer B.Cu) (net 28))
 (segment (start 90.5 80.335002) (end 90.5 73.5) (width 0.25) (layer B.Cu) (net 28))
 (via (at 90.5 80.335002) (size 0.75) (drill 0.4) (layers F.Cu B.Cu) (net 28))
 (segment (start 96 82.5) (end 96 88) (width 0.25) (layer F.Cu) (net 28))
 (segment (start 97.5 89.5) (end 101 89.5) (width 0.25) (layer F.Cu) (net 28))
 (segment (start 90.5 80.335002) (end 91.664998 81.5) (width 0.25) (layer F.Cu) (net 28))
 (segment (start 95 81.5) (end 96 82.5) (width 0.25) (layer F.Cu) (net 28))
 (segment (start 96 88) (end 97.5 89.5) (width 0.25) (layer F.Cu) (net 28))
 (segment (start 91.664998 81.5) (end 95 81.5) (width 0.25) (layer F.Cu) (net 28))
 (segment (start 105 86) (end 109.5 81.5) (width 0.25) (layer F.Cu) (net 9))
 (segment (start 103.93 77.31) (end 101 80.24) (width 0.25) (layer F.Cu) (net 26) (status 10))
 (segment (start 101 80.24) (end 101 85.75) (width 0.25) (layer F.Cu) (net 26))
 (segment (start 90 97.1524) (end 90 97) (width 0.5) (layer B.Cu) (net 14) (status 30))
 (segment (start 109 66.4) (end 106.5 68.9) (width 0.5) (layer B.Cu) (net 14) (status 10))
 (segment (start 82.420001 63.259999) (end 81.07 64.61) (width 0.5) (layer B.Cu) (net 14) (status 20))
 (segment (start 105.859999 63.259999) (end 82.420001 63.259999) (width 0.5) (layer B.Cu) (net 14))
 (segment (start 109 66.4) (end 105.859999 63.259999) (width 0.5) (layer B.Cu) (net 14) (status 10))
 (segment (start 106.5 68.9) (end 106.5 92) (width 0.5) (layer B.Cu) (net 14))
 (segment (start 106.5 92) (end 99.5 99) (width 0.5) (layer B.Cu) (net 14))
 (segment (start 91.8476 99) (end 90 97.1524) (width 0.5) (layer B.Cu) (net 14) (status 20))
 (segment (start 99.5 99) (end 91.8476 99) (width 0.5) (layer B.Cu) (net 14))
 (segment (start 87.15 97) (end 90 97) (width 0.5) (layer F.Cu) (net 14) (status 20))
 (segment (start 85 93.5) (end 85 94.85) (width 0.5) (layer F.Cu) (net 14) (status 10))
 (segment (start 85 94.85) (end 87.15 97) (width 0.5) (layer F.Cu) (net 14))
 (segment (start 81.07 77.31) (end 87.54 83.78) (width 0.25) (layer B.Cu) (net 25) (status 10))
 (segment (start 87.54 83.78) (end 87.54 93.5) (width 0.25) (layer B.Cu) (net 25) (status 20))
 (segment (start 81.07 74.77) (end 90.08 83.78) (width 0.25) (layer B.Cu) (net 27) (status 10))
 (segment (start 90.08 83.78) (end 90.08 93.5) (width 0.25) (layer B.Cu) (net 27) (status 20))
 (segment (start 103.93 79.85) (end 95.16 88.62) (width 0.25) (layer B.Cu) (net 24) (status 10))
 (segment (start 95.16 88.62) (end 95.16 93.5) (width 0.25) (layer B.Cu) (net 24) (status 20))
 (segment (start 92.54 95.734) (end 92.54 97) (width 0.25) (layer B.Cu) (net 15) (status 20))
 (segment (start 91.444999 94.638999) (end 92.54 95.734) (width 0.25) (layer B.Cu) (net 15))
 (segment (start 91.444999 79.635001) (end 91.444999 94.638999) (width 0.25) (layer B.Cu) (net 15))
 (segment (start 101.39 69.69) (end 103.93 69.69) (width 0.25) (layer B.Cu) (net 15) (status 20))
 (segment (start 91.444999 79.635001) (end 101.39 69.69) (width 0.25) (layer B.Cu) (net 15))
 (segment (start 103.93 64.61) (end 105.155001 65.835001) (width 0.25) (layer B.Cu) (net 29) (status 10))
 (segment (start 105.155001 65.835001) (end 105.155001 86.044999) (width 0.25) (layer B.Cu) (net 29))
 (segment (start 105.155001 86.044999) (end 97.7 93.5) (width 0.25) (layer B.Cu) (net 29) (status 20))
 (segment (start 123.5 86.62) (end 123.5 90.5) (width 2) (layer B.Cu) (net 23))
 (segment (start 123.5 90.5) (end 123.5 91) (width 2) (layer B.Cu) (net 23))
 (segment (start 125 92.5) (end 135.5 92.5) (width 2) (layer B.Cu) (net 23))
 (segment (start 123.5 91) (end 125 92.5) (width 2) (layer B.Cu) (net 23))
 (segment (start 128.5 87.5) (end 128 87) (width 2) (layer F.Cu) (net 1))
 (segment (start 135.5 87.5) (end 128.5 87.5) (width 2) (layer F.Cu) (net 1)))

